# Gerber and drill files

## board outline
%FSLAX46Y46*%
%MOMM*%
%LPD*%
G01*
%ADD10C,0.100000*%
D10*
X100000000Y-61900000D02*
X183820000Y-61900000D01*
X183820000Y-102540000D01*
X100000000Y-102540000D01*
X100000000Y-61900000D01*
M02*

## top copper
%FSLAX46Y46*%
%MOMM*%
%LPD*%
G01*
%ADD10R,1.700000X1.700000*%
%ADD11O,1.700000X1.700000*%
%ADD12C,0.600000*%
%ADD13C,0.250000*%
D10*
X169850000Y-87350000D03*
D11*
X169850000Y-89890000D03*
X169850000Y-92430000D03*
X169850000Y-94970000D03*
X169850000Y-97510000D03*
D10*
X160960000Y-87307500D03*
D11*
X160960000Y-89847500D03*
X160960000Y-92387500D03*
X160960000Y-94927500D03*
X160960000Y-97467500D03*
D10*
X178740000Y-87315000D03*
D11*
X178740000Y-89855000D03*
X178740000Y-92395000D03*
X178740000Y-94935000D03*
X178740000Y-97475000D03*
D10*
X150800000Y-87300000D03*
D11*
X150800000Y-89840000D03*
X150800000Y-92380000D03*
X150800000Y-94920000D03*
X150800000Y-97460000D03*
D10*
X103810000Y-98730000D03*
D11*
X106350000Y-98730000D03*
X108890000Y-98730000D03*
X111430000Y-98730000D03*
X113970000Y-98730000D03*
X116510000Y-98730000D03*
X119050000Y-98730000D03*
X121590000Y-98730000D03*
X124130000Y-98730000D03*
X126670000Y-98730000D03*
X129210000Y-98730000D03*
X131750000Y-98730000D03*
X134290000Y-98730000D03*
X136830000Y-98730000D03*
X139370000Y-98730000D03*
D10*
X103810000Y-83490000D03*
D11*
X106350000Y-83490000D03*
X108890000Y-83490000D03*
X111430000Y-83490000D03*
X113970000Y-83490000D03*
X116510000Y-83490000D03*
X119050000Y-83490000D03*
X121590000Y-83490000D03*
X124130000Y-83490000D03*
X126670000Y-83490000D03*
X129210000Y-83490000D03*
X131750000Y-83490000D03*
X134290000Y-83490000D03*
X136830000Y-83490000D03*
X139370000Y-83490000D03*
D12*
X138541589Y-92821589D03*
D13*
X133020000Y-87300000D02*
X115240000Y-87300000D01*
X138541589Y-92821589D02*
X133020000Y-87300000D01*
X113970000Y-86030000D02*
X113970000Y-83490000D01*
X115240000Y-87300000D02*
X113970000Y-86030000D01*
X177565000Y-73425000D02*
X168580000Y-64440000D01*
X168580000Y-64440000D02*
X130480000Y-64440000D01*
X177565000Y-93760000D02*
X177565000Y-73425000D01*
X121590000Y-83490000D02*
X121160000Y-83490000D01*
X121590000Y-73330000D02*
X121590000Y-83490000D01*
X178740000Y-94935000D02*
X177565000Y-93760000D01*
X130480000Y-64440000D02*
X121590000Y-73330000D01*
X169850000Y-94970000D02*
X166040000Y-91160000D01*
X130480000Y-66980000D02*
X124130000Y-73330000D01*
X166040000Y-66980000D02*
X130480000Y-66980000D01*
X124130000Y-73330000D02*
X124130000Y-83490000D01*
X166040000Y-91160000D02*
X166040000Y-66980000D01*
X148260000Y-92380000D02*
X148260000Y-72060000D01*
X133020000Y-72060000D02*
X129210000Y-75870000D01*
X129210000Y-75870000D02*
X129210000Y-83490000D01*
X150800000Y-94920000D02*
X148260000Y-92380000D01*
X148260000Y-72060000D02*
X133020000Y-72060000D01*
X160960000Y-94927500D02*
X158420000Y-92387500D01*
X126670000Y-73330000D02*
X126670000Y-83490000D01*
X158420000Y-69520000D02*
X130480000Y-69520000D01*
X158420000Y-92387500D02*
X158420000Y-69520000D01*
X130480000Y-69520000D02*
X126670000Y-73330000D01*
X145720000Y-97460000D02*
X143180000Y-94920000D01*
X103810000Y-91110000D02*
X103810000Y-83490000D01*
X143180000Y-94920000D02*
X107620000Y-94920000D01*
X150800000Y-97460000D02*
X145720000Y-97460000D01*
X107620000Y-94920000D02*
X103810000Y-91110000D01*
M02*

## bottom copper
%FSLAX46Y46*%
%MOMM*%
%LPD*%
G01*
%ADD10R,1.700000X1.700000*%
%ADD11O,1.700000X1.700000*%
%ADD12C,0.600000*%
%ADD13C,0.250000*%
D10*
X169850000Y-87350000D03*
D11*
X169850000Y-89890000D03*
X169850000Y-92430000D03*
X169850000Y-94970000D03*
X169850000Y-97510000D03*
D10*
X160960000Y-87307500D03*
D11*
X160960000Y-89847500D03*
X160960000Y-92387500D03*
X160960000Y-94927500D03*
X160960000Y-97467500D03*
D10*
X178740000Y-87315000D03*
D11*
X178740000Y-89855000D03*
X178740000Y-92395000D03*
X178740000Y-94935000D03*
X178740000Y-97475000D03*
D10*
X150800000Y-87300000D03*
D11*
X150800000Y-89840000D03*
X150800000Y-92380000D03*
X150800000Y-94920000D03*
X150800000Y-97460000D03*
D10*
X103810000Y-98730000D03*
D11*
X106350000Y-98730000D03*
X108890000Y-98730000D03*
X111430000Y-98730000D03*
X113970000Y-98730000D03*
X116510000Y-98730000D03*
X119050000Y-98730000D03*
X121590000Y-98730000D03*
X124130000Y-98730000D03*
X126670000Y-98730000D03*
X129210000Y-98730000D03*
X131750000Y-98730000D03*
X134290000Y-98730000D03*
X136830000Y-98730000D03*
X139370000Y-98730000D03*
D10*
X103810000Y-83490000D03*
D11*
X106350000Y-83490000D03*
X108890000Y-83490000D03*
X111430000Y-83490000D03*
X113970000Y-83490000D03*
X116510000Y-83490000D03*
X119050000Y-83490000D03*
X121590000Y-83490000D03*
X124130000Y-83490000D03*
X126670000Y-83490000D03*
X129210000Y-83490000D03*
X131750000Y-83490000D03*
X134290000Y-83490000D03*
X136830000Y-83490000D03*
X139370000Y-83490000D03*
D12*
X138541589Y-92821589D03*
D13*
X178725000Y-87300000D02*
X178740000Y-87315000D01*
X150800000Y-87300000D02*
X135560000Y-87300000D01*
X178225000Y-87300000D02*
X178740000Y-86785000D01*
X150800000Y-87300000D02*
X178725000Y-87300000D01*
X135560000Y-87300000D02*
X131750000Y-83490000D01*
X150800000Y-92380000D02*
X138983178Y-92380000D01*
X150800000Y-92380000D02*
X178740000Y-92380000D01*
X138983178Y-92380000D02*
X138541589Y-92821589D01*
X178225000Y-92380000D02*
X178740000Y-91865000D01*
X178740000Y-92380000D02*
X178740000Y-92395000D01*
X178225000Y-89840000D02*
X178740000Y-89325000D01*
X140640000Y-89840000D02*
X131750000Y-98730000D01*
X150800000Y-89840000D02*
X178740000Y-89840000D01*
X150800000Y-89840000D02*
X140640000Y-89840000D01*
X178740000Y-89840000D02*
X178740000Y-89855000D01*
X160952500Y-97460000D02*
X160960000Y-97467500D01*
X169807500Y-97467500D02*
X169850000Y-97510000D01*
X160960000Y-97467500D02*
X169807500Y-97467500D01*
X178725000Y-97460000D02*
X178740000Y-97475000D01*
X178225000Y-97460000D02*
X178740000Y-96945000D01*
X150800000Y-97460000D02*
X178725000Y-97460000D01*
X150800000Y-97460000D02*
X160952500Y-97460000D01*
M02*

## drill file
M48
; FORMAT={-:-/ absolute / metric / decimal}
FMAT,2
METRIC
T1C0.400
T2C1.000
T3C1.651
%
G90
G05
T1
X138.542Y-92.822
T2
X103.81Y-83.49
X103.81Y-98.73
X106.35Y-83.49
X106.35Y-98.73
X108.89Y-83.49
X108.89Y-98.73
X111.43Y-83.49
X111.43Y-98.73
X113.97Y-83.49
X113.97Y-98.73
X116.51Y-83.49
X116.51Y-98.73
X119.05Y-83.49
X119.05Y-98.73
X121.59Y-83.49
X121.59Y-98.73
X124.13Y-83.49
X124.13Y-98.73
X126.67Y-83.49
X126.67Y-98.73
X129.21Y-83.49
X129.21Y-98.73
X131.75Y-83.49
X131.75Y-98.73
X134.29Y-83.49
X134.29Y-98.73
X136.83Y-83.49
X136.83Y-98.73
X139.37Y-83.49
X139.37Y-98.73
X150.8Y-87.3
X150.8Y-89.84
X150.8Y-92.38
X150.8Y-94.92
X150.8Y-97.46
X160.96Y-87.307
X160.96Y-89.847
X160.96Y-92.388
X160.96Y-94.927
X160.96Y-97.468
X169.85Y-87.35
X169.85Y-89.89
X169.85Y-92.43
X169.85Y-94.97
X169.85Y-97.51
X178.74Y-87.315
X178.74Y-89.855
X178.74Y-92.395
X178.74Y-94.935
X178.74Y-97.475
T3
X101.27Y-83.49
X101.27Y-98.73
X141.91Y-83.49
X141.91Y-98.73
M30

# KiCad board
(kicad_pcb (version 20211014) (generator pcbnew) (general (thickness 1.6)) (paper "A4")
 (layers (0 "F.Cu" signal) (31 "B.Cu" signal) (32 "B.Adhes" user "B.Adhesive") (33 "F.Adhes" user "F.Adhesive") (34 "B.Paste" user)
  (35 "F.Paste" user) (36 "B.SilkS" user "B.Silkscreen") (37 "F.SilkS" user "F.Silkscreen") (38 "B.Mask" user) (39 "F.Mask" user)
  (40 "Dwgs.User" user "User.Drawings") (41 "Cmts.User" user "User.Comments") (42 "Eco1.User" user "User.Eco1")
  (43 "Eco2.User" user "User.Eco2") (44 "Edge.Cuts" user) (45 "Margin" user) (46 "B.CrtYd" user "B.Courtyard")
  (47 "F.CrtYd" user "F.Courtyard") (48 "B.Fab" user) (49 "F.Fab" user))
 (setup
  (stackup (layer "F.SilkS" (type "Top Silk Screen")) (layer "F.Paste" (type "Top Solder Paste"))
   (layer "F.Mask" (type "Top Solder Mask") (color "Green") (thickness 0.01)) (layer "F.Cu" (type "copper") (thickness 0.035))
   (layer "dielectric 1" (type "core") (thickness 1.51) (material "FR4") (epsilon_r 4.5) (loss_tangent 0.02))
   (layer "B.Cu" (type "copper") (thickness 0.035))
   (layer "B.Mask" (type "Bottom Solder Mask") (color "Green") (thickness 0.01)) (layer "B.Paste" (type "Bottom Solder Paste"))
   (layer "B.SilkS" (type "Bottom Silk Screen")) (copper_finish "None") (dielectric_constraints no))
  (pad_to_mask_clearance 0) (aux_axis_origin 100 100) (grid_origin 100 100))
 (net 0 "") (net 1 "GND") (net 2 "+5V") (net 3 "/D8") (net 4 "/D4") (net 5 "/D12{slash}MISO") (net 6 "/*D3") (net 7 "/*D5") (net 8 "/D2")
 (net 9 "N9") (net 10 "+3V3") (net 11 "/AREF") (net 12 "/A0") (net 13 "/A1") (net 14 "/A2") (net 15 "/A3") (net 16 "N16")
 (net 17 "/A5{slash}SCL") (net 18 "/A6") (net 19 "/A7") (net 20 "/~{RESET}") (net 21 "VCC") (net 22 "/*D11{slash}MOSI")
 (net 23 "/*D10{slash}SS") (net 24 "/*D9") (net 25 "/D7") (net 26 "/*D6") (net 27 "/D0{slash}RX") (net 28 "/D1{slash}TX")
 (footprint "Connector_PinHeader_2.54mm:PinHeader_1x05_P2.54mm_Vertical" (layer "F.Cu") (at 169.85 87.35)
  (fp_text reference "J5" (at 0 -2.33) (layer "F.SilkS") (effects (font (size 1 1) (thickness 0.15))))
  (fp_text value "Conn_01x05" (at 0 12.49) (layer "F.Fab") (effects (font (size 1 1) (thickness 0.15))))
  (pad "1" thru_hole rect (at 0 0) (size 1.7 1.7) (drill 1) (layers *.Cu *.Mask) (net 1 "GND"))
  (pad "2" thru_hole oval (at 0 2.54) (size 1.7 1.7) (drill 1) (layers *.Cu *.Mask) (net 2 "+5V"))
  (pad "3" thru_hole oval (at 0 5.08) (size 1.7 1.7) (drill 1) (layers *.Cu *.Mask) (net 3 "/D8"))
  (pad "4" thru_hole oval (at 0 7.62) (size 1.7 1.7) (drill 1) (layers *.Cu *.Mask) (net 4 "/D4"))
  (pad "5" thru_hole oval (at 0 10.16) (size 1.7 1.7) (drill 1) (layers *.Cu *.Mask) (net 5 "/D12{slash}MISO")))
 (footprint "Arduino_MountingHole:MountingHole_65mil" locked (layer "F.Cu") (at 101.27 83.49)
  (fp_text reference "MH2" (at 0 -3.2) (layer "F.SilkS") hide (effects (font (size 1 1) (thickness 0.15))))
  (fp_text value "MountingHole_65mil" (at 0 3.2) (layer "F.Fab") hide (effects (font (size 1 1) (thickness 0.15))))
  (pad "" np_thru_hole circle locked (at 0 0) (size 1.651 1.651) (drill 1.651) (layers F&B.Cu *.Mask)))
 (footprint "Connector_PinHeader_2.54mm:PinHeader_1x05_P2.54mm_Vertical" (layer "F.Cu") (at 160.96 87.3075)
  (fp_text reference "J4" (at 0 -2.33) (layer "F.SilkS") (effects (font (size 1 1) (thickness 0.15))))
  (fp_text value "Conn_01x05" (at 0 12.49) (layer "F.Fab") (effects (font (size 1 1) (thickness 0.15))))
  (pad "1" thru_hole rect (at 0 0) (size 1.7 1.7) (drill 1) (layers *.Cu *.Mask) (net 1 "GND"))
  (pad "2" thru_hole oval (at 0 2.54) (size 1.7 1.7) (drill 1) (layers *.Cu *.Mask) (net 2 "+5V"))
  (pad "3" thru_hole oval (at 0 5.08) (size 1.7 1.7) (drill 1) (layers *.Cu *.Mask) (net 3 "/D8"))
  (pad "4" thru_hole oval (at 0 7.62) (size 1.7 1.7) (drill 1) (layers *.Cu *.Mask) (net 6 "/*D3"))
  (pad "5" thru_hole oval (at 0 10.16) (size 1.7 1.7) (drill 1) (layers *.Cu *.Mask) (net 5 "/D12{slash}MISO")))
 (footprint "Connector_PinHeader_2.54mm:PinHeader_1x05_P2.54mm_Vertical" (layer "F.Cu") (at 178.74 87.315)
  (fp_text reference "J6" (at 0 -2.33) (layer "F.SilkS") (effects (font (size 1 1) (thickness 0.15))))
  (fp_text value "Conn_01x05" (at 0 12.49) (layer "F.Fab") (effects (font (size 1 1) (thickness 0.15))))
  (pad "1" thru_hole rect (at 0 0) (size 1.7 1.7) (drill 1) (layers *.Cu *.Mask) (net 1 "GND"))
  (pad "2" thru_hole oval (at 0 2.54) (size 1.7 1.7) (drill 1) (layers *.Cu *.Mask) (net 2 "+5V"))
  (pad "3" thru_hole oval (at 0 5.08) (size 1.7 1.7) (drill 1) (layers *.Cu *.Mask) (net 3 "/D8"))
  (pad "4" thru_hole oval (at 0 7.62) (size 1.7 1.7) (drill 1) (layers *.Cu *.Mask) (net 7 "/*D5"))
  (pad "5" thru_hole oval (at 0 10.16) (size 1.7 1.7) (drill 1) (layers *.Cu *.Mask) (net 5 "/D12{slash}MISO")))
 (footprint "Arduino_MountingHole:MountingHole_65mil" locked (layer "F.Cu") (at 141.91 98.73)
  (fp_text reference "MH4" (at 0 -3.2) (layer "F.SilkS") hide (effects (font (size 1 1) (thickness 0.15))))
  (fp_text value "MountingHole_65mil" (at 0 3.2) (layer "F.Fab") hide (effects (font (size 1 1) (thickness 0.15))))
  (pad "" np_thru_hole circle locked (at 0 0) (size 1.651 1.651) (drill 1.651) (layers F&B.Cu *.Mask)))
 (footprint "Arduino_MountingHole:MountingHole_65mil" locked (layer "F.Cu") (at 101.27 98.73)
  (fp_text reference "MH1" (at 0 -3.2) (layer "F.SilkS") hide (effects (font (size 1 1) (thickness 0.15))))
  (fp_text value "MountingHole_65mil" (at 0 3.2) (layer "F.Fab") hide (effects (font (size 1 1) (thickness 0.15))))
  (pad "" np_thru_hole circle locked (at 0 0) (size 1.651 1.651) (drill 1.651) (layers F&B.Cu *.Mask)))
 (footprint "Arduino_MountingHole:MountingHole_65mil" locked (layer "F.Cu") (at 141.91 83.49)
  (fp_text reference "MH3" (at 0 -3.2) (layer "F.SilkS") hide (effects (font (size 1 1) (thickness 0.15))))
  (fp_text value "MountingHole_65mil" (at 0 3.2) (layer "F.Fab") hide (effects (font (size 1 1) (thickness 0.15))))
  (pad "" np_thru_hole circle locked (at 0 0) (size 1.651 1.651) (drill 1.651) (layers F&B.Cu *.Mask)))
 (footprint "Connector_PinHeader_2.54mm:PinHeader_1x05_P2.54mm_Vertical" (layer "F.Cu") (at 150.8 87.3)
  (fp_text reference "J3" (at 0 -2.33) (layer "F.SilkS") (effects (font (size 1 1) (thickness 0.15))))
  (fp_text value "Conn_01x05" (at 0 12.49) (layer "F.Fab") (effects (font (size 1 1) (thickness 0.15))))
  (pad "1" thru_hole rect (at 0 0) (size 1.7 1.7) (drill 1) (layers *.Cu *.Mask) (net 1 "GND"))
  (pad "2" thru_hole oval (at 0 2.54) (size 1.7 1.7) (drill 1) (layers *.Cu *.Mask) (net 2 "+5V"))
  (pad "3" thru_hole oval (at 0 5.08) (size 1.7 1.7) (drill 1) (layers *.Cu *.Mask) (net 3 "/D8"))
  (pad "4" thru_hole oval (at 0 7.62) (size 1.7 1.7) (drill 1) (layers *.Cu *.Mask) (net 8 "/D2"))
  (pad "5" thru_hole oval (at 0 10.16) (size 1.7 1.7) (drill 1) (layers *.Cu *.Mask) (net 5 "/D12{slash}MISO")))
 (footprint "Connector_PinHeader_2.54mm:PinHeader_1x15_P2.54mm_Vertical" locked (layer "B.Cu") (at 103.81 98.73 -90)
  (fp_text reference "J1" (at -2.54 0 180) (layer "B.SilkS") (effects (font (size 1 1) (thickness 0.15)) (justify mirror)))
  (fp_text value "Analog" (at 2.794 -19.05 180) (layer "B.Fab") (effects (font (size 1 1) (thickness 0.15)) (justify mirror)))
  (pad "1" thru_hole rect locked (at 0 0 270) (size 1.7 1.7) (drill 1) (layers *.Cu *.Mask) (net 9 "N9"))
  (pad "2" thru_hole oval locked (at 0 -2.54 270) (size 1.7 1.7) (drill 1) (layers *.Cu *.Mask) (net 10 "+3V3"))
  (pad "3" thru_hole oval locked (at 0 -5.08 270) (size 1.7 1.7) (drill 1) (layers *.Cu *.Mask) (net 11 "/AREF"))
  (pad "4" thru_hole oval locked (at 0 -7.62 270) (size 1.7 1.7) (drill 1) (layers *.Cu *.Mask) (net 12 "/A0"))
  (pad "5" thru_hole oval locked (at 0 -10.16 270) (size 1.7 1.7) (drill 1) (layers *.Cu *.Mask) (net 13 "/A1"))
  (pad "6" thru_hole oval locked (at 0 -12.7 270) (size 1.7 1.7) (drill 1) (layers *.Cu *.Mask) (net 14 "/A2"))
  (pad "7" thru_hole oval locked (at 0 -15.24 270) (size 1.7 1.7) (drill 1) (layers *.Cu *.Mask) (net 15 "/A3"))
  (pad "8" thru_hole oval locked (at 0 -17.78 270) (size 1.7 1.7) (drill 1) (layers *.Cu *.Mask) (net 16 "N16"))
  (pad "9" thru_hole oval locked (at 0 -20.32 270) (size 1.7 1.7) (drill 1) (layers *.Cu *.Mask) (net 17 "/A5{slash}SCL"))
  (pad "10" thru_hole oval locked (at 0 -22.86 270) (size 1.7 1.7) (drill 1) (layers *.Cu *.Mask) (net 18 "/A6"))
  (pad "11" thru_hole oval locked (at 0 -25.4 270) (size 1.7 1.7) (drill 1) (layers *.Cu *.Mask) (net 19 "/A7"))
  (pad "12" thru_hole oval locked (at 0 -27.94 270) (size 1.7 1.7) (drill 1) (layers *.Cu *.Mask) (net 2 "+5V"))
  (pad "13" thru_hole oval locked (at 0 -30.48 270) (size 1.7 1.7) (drill 1) (layers *.Cu *.Mask) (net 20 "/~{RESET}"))
  (pad "14" thru_hole oval locked (at 0 -33.02 270) (size 1.7 1.7) (drill 1) (layers *.Cu *.Mask) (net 1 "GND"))
  (pad "15" thru_hole oval locked (at 0 -35.56 270) (size 1.7 1.7) (drill 1) (layers *.Cu *.Mask) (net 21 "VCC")))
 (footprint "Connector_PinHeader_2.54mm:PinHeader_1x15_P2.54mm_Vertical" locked (layer "B.Cu") (at 103.81 83.49 -90)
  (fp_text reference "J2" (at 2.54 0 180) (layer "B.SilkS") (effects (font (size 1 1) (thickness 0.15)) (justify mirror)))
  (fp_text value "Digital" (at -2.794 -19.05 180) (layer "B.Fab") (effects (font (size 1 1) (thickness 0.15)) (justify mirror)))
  (pad "1" thru_hole rect locked (at 0 0 270) (size 1.7 1.7) (drill 1) (layers *.Cu *.Mask) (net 5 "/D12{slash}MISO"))
  (pad "2" thru_hole oval locked (at 0 -2.54 270) (size 1.7 1.7) (drill 1) (layers *.Cu *.Mask) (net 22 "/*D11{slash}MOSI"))
  (pad "3" thru_hole oval locked (at 0 -5.08 270) (size 1.7 1.7) (drill 1) (layers *.Cu *.Mask) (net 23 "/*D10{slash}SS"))
  (pad "4" thru_hole oval locked (at 0 -7.62 270) (size 1.7 1.7) (drill 1) (layers *.Cu *.Mask) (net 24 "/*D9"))
  (pad "5" thru_hole oval locked (at 0 -10.16 270) (size 1.7 1.7) (drill 1) (layers *.Cu *.Mask) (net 3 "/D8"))
  (pad "6" thru_hole oval locked (at 0 -12.7 270) (size 1.7 1.7) (drill 1) (layers *.Cu *.Mask) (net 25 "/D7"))
  (pad "7" thru_hole oval locked (at 0 -15.24 270) (size 1.7 1.7) (drill 1) (layers *.Cu *.Mask) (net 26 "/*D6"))
  (pad "8" thru_hole oval locked (at 0 -17.78 270) (size 1.7 1.7) (drill 1) (layers *.Cu *.Mask) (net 7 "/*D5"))
  (pad "9" thru_hole oval locked (at 0 -20.32 270) (size 1.7 1.7) (drill 1) (layers *.Cu *.Mask) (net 4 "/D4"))
  (pad "10" thru_hole oval locked (at 0 -22.86 270) (size 1.7 1.7) (drill 1) (layers *.Cu *.Mask) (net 6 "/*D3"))
  (pad "11" thru_hole oval locked (at 0 -25.4 270) (size 1.7 1.7) (drill 1) (layers *.Cu *.Mask) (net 8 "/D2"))
  (pad "12" thru_hole oval locked (at 0 -27.94 270) (size 1.7 1.7) (drill 1) (layers *.Cu *.Mask) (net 1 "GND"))
  (pad "13" thru_hole oval locked (at 0 -30.48 270) (size 1.7 1.7) (drill 1) (layers *.Cu *.Mask) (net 20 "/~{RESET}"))
  (pad "14" thru_hole oval locked (at 0 -33.02 270) (size 1.7 1.7) (drill 1) (layers *.Cu *.Mask) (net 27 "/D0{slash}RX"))
  (pad "15" thru_hole oval locked (at 0 -35.56 270) (size 1.7 1.7) (drill 1) (layers *.Cu *.Mask) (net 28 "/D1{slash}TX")))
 (gr_rect (start 100 61.9) (end 183.82 102.54) (layer "Edge.Cuts") (width 0.1) (fill none))
 (segment (start 178.725 87.3) (end 178.74 87.315) (width 0.25) (layer "B.Cu") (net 1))
 (segment (start 150.8 87.3) (end 135.56 87.3) (width 0.25) (layer "B.Cu") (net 1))
 (segment (start 178.225 87.3) (end 178.74 86.785) (width 0.25) (layer "B.Cu") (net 1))
 (segment (start 150.8 87.3) (end 178.725 87.3) (width 0.25) (layer "B.Cu") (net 1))
 (segment (start 135.56 87.3) (end 131.75 83.49) (width 0.25) (layer "B.Cu") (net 1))
 (segment (start 133.02 87.3) (end 115.24 87.3) (width 0.25) (layer "F.Cu") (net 3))
 (segment (start 138.541589 92.821589) (end 133.02 87.3) (width 0.25) (layer "F.Cu") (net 3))
 (segment (start 113.97 86.03) (end 113.97 83.49) (width 0.25) (layer "F.Cu") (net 3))
 (segment (start 115.24 87.3) (end 113.97 86.03) (width 0.25) (layer "F.Cu") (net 3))
 (via (at 138.541589 92.821589) (size 0.6) (drill 0.4) (layers "F.Cu" "B.Cu") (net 3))
 (segment (start 150.8 92.38) (end 138.983178 92.38) (width 0.25) (layer "B.Cu") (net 3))
 (segment (start 150.8 92.38) (end 178.74 92.38) (width 0.25) (layer "B.Cu") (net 3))
 (segment (start 138.983178 92.38) (end 138.541589 92.821589) (width 0.25) (layer "B.Cu") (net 3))
 (segment (start 178.225 92.38) (end 178.74 91.865) (width 0.25) (layer "B.Cu") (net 3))
 (segment (start 178.74 92.38) (end 178.74 92.395) (width 0.25) (layer "B.Cu") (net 3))
 (segment (start 177.565 73.425) (end 168.58 64.44) (width 0.25) (layer "F.Cu") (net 7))
 (segment (start 168.58 64.44) (end 130.48 64.44) (width 0.25) (layer "F.Cu") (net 7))
 (segment (start 177.565 93.76) (end 177.565 73.425) (width 0.25) (layer "F.Cu") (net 7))
 (segment (start 121.59 83.49) (end 121.16 83.49) (width 0.25) (layer "F.Cu") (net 7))
 (segment (start 121.59 73.33) (end 121.59 83.49) (width 0.25) (layer "F.Cu") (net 7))
 (segment (start 178.74 94.935) (end 177.565 93.76) (width 0.25) (layer "F.Cu") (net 7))
 (segment (start 130.48 64.44) (end 121.59 73.33) (width 0.25) (layer "F.Cu") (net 7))
 (segment (start 169.85 94.97) (end 166.04 91.16) (width 0.25) (layer "F.Cu") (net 4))
 (segment (start 130.48 66.98) (end 124.13 73.33) (width 0.25) (layer "F.Cu") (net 4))
 (segment (start 166.04 66.98) (end 130.48 66.98) (width 0.25) (layer "F.Cu") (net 4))
 (segment (start 124.13 73.33) (end 124.13 83.49) (width 0.25) (layer "F.Cu") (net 4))
 (segment (start 166.04 91.16) (end 166.04 66.98) (width 0.25) (layer "F.Cu") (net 4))
 (segment (start 178.225 89.84) (end 178.74 89.325) (width 0.25) (layer "B.Cu") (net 2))
 (segment (start 140.64 89.84) (end 131.75 98.73) (width 0.25) (layer "B.Cu") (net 2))
 (segment (start 150.8 89.84) (end 178.74 89.84) (width 0.25) (layer "B.Cu") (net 2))
 (segment (start 150.8 89.84) (end 140.64 89.84) (width 0.25) (layer "B.Cu") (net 2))
 (segment (start 178.74 89.84) (end 178.74 89.855) (width 0.25) (layer "B.Cu") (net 2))
 (segment (start 148.26 92.38) (end 148.26 72.06) (width 0.25) (layer "F.Cu") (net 8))
 (segment (start 133.02 72.06) (end 129.21 75.87) (width 0.25) (layer "F.Cu") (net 8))
 (segment (start 129.21 75.87) (end 129.21 83.49) (width 0.25) (layer "F.Cu") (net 8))
 (segment (start 150.8 94.92) (end 148.26 92.38) (width 0.25) (layer "F.Cu") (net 8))
 (segment (start 148.26 72.06) (end 133.02 72.06) (width 0.25) (layer "F.Cu") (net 8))
 (segment (start 160.96 94.9275) (end 158.42 92.3875) (width 0.25) (layer "F.Cu") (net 6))
 (segment (start 126.67 73.33) (end 126.67 83.49) (width 0.25) (layer "F.Cu") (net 6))
 (segment (start 158.42 69.52) (end 130.48 69.52) (width 0.25) (layer "F.Cu") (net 6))
 (segment (start 158.42 92.3875) (end 158.42 69.52) (width 0.25) (layer "F.Cu") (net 6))
 (segment (start 130.48 69.52) (end 126.67 73.33) (width 0.25) (layer "F.Cu") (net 6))
 (segment (start 145.72 97.46) (end 143.18 94.92) (width 0.25) (layer "F.Cu") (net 5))
 (segment (start 103.81 91.11) (end 103.81 83.49) (width 0.25) (layer "F.Cu") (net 5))
 (segment (start 143.18 94.92) (end 107.62 94.92) (width 0.25) (layer "F.Cu") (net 5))
 (segment (start 150.8 97.46) (end 145.72 97.46) (width 0.25) (layer "F.Cu") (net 5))
 (segment (start 107.62 94.92) (end 103.81 91.11) (width 0.25) (layer "F.Cu") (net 5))
 (segment (start 160.9525 97.46) (end 160.96 97.4675) (width 0.25) (layer "B.Cu") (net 5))
 (segment (start 169.8075 97.4675) (end 169.85 97.51) (width 0.25) (layer "B.Cu") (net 5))
 (segment (start 160.96 97.4675) (end 169.8075 97.4675) (width 0.25) (layer "B.Cu") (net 5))
 (segment (start 178.725 97.46) (end 178.74 97.475) (width 0.25) (layer "B.Cu") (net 5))
 (segment (start 178.225 97.46) (end 178.74 96.945) (width 0.25) (layer "B.Cu") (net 5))
 (segment (start 150.8 97.46) (end 178.725 97.46) (width 0.25) (layer "B.Cu") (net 5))
 (segment (start 150.8 97.46) (end 160.9525 97.46) (width 0.25) (layer "B.Cu") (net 5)))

